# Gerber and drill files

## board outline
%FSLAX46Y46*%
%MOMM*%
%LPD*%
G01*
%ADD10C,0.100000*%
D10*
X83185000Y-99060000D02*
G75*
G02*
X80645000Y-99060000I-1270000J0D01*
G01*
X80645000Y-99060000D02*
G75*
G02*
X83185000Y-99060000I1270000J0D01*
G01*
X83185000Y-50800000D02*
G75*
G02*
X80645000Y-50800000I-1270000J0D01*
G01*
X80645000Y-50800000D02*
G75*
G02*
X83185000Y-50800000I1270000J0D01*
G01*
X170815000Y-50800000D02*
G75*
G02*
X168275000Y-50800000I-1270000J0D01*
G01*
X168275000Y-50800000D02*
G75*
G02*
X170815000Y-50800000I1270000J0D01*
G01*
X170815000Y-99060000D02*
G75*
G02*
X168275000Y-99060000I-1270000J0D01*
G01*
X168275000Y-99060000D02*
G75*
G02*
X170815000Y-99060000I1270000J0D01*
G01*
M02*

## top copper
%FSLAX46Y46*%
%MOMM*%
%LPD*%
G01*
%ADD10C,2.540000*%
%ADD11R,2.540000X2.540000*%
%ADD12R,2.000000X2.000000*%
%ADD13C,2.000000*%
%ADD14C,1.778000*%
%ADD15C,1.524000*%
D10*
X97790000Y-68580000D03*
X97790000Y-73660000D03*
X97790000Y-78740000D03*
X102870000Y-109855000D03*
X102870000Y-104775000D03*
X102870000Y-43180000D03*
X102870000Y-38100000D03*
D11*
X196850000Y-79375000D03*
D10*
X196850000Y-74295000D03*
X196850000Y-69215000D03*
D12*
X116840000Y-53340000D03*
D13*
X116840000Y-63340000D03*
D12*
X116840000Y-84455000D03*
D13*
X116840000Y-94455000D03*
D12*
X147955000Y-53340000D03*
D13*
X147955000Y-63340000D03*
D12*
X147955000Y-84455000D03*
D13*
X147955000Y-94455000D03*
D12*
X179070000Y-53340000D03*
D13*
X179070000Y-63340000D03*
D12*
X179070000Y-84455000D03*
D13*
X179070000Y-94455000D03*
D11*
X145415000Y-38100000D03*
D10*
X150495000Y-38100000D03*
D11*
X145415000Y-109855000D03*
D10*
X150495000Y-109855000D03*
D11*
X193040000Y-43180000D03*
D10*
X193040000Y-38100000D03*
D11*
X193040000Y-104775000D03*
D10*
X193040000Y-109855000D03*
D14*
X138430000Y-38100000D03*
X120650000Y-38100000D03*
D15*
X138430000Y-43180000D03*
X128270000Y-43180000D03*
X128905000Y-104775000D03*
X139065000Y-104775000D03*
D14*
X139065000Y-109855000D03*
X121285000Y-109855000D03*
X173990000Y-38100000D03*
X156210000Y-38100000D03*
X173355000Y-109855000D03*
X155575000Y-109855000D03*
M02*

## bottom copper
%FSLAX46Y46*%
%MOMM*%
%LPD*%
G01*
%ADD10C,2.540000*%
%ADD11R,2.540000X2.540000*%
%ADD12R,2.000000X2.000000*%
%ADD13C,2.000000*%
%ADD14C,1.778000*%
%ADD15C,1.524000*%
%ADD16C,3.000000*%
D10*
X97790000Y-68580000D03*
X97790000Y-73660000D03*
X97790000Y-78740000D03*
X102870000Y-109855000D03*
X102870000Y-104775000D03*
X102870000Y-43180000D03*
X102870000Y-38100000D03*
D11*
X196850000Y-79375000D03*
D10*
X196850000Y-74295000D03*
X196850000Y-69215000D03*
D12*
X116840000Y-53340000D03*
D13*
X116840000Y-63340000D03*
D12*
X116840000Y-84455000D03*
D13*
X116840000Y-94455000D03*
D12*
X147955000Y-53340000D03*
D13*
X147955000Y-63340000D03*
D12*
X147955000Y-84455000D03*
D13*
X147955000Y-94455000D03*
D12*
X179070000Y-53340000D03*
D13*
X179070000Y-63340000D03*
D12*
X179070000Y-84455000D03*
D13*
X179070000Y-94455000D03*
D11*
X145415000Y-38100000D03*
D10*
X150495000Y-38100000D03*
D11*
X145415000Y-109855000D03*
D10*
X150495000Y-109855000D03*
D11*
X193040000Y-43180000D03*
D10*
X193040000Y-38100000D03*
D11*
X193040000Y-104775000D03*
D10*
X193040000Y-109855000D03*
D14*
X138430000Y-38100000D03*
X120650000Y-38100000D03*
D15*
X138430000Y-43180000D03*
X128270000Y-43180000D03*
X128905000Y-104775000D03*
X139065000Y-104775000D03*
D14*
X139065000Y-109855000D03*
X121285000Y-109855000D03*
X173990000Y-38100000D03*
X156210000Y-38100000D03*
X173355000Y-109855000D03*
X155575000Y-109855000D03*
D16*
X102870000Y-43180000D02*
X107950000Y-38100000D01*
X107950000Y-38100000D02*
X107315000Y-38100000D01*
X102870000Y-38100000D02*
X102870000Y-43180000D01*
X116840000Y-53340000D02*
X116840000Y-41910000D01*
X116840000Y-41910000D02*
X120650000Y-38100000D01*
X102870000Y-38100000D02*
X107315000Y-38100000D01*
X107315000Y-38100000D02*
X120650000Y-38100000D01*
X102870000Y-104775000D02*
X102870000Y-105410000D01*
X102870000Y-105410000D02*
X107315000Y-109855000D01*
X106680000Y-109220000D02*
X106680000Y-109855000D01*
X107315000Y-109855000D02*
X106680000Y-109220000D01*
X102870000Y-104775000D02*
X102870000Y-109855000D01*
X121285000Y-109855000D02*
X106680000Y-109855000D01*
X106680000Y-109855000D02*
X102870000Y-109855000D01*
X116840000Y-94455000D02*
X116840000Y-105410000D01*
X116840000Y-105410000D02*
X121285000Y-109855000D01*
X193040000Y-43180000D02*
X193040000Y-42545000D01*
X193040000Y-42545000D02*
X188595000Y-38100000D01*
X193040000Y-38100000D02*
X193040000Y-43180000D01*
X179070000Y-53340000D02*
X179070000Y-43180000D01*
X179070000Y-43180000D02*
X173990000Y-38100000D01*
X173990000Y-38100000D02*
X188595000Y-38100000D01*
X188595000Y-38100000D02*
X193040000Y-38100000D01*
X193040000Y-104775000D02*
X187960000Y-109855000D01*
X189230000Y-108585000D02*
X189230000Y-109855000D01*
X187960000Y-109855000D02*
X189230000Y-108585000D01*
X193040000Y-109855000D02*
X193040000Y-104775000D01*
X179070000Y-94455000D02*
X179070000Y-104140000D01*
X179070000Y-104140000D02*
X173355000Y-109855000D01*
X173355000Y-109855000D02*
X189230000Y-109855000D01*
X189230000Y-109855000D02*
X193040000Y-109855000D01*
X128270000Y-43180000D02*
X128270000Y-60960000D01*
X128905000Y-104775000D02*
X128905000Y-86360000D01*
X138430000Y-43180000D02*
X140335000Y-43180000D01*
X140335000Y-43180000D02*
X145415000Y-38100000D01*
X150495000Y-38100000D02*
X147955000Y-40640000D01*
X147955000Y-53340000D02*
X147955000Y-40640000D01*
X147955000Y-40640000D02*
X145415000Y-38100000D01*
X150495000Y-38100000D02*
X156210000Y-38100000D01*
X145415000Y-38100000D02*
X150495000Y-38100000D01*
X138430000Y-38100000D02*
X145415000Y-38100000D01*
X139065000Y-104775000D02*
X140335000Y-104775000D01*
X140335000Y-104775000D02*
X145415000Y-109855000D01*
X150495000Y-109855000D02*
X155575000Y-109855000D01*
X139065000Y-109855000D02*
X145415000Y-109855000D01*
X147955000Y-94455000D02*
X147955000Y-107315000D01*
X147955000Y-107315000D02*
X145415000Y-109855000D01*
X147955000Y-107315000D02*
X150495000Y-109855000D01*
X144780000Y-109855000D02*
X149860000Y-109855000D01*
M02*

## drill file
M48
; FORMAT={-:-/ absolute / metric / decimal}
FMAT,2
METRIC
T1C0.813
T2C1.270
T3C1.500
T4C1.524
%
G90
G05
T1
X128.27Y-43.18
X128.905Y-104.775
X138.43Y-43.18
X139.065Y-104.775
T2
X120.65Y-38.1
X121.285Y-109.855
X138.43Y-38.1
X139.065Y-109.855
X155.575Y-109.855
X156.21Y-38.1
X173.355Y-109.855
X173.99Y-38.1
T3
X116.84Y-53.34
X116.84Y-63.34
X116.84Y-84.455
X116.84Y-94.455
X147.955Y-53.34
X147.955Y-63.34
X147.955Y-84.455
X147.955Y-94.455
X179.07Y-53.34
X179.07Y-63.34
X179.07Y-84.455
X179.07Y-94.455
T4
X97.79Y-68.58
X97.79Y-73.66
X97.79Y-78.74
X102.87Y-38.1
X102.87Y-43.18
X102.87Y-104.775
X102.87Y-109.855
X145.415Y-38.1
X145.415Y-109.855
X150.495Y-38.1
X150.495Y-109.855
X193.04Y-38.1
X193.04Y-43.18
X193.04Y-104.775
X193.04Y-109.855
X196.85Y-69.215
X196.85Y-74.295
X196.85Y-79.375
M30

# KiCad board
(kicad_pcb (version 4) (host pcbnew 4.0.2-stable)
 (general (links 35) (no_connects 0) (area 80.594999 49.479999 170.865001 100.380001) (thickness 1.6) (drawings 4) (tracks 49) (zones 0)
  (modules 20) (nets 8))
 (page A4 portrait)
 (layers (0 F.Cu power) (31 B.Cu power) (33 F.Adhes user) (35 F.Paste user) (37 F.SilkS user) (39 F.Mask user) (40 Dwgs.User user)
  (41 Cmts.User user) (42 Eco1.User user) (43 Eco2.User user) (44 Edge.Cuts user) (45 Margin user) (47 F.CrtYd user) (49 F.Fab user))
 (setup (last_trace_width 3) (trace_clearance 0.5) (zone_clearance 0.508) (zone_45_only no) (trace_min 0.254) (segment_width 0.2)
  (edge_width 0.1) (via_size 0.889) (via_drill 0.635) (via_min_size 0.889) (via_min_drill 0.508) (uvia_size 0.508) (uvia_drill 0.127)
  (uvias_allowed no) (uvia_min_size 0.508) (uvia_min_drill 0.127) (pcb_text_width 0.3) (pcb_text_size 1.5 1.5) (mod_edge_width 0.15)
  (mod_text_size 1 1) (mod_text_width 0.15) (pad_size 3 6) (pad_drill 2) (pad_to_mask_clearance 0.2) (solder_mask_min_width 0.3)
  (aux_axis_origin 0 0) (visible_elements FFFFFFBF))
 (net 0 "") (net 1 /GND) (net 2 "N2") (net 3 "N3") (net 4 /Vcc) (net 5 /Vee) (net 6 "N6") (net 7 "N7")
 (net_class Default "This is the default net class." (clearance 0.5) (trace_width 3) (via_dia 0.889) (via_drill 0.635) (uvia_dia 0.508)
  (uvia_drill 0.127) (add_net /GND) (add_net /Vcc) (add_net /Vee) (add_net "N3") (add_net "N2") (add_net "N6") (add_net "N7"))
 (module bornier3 (layer F.Cu) (at 97.79 73.66 270)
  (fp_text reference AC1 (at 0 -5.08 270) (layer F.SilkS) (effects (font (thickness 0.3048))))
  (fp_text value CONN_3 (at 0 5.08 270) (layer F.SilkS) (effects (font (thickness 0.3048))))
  (pad 1 thru_hole circle (at -5.08 0 270) (size 2.54 2.54) (drill 1.524) (layers *.Cu *.Mask F.SilkS) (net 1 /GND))
  (pad 2 thru_hole circle (at 0 0 270) (size 2.54 2.54) (drill 1.524) (layers *.Cu *.Mask F.SilkS) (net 1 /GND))
  (pad 3 thru_hole circle (at 5.08 0 270) (size 2.54 2.54) (drill 1.524) (layers *.Cu *.Mask F.SilkS) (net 1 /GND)))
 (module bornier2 (layer F.Cu) (at 102.87 107.315 90)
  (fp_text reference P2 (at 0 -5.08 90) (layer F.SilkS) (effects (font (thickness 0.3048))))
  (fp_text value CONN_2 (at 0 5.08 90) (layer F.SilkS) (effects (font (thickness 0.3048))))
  (pad 1 thru_hole circle (at -2.54 0 90) (size 2.54 2.54) (drill 1.524) (layers *.Cu *.Mask F.SilkS) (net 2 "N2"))
  (pad 2 thru_hole circle (at 2.54 0 90) (size 2.54 2.54) (drill 1.524) (layers *.Cu *.Mask F.SilkS) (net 2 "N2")))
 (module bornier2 (layer F.Cu) (at 102.87 40.64 90)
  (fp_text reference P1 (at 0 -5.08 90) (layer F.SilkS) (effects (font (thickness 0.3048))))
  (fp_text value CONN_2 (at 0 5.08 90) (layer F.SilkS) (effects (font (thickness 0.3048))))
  (pad 1 thru_hole circle (at -2.54 0 90) (size 2.54 2.54) (drill 1.524) (layers *.Cu *.Mask F.SilkS) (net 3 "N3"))
  (pad 2 thru_hole circle (at 2.54 0 90) (size 2.54 2.54) (drill 1.524) (layers *.Cu *.Mask F.SilkS) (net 3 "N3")))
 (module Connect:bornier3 (layer F.Cu) (at 196.85 74.295 90)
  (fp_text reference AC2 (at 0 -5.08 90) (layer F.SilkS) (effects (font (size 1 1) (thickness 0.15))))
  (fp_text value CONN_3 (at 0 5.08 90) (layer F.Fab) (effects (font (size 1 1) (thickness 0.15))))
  (pad 1 thru_hole rect (at -5.08 0 90) (size 2.54 2.54) (drill 1.524) (layers *.Cu *.Mask F.SilkS) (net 1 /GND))
  (pad 2 thru_hole circle (at 0 0 90) (size 2.54 2.54) (drill 1.524) (layers *.Cu *.Mask F.SilkS) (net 1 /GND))
  (pad 3 thru_hole circle (at 5.08 0 90) (size 2.54 2.54) (drill 1.524) (layers *.Cu *.Mask F.SilkS) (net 1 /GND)))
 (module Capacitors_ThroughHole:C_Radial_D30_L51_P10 (layer F.Cu) (at 116.84 53.34 270)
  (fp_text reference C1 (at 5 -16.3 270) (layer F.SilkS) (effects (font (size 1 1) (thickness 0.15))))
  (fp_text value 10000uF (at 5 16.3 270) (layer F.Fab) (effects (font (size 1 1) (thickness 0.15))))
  (pad 1 thru_hole rect (at 0 0 270) (size 2 2) (drill 1.5) (layers *.Cu *.Mask F.SilkS) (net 3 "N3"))
  (pad 2 thru_hole circle (at 10 0 270) (size 2 2) (drill 1.5) (layers *.Cu *.Mask F.SilkS) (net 1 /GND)))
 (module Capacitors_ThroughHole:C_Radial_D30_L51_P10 (layer F.Cu) (at 116.84 84.455 270)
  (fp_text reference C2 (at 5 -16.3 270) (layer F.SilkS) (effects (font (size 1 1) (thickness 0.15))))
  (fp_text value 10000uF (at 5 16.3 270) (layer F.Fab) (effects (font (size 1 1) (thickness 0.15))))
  (pad 1 thru_hole rect (at 0 0 270) (size 2 2) (drill 1.5) (layers *.Cu *.Mask F.SilkS) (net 1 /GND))
  (pad 2 thru_hole circle (at 10 0 270) (size 2 2) (drill 1.5) (layers *.Cu *.Mask F.SilkS) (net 2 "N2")))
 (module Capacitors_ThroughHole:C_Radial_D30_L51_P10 (layer F.Cu) (at 147.955 53.34 270)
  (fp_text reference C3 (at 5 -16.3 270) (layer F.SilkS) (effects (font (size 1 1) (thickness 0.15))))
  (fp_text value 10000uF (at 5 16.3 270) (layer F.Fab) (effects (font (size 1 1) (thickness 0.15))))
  (pad 1 thru_hole rect (at 0 0 270) (size 2 2) (drill 1.5) (layers *.Cu *.Mask F.SilkS) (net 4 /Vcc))
  (pad 2 thru_hole circle (at 10 0 270) (size 2 2) (drill 1.5) (layers *.Cu *.Mask F.SilkS) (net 1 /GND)))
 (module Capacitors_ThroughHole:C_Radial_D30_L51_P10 (layer F.Cu) (at 147.955 84.455 270)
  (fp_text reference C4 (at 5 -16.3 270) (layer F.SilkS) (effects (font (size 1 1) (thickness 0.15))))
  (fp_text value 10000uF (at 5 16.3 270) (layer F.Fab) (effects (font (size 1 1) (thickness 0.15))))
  (pad 1 thru_hole rect (at 0 0 270) (size 2 2) (drill 1.5) (layers *.Cu *.Mask F.SilkS) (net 1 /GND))
  (pad 2 thru_hole circle (at 10 0 270) (size 2 2) (drill 1.5) (layers *.Cu *.Mask F.SilkS) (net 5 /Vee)))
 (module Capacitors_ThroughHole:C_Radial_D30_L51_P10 (layer F.Cu) (at 179.07 53.34 270)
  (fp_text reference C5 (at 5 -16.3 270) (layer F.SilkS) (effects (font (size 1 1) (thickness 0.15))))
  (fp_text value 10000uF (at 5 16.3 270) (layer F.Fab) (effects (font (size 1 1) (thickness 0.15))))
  (pad 1 thru_hole rect (at 0 0 270) (size 2 2) (drill 1.5) (layers *.Cu *.Mask F.SilkS) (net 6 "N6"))
  (pad 2 thru_hole circle (at 10 0 270) (size 2 2) (drill 1.5) (layers *.Cu *.Mask F.SilkS) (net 1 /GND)))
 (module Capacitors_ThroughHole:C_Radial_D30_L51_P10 (layer F.Cu) (at 179.07 84.455 270)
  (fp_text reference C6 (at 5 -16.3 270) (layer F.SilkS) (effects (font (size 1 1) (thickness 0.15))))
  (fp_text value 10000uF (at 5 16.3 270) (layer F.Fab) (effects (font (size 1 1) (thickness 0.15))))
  (pad 1 thru_hole rect (at 0 0 270) (size 2 2) (drill 1.5) (layers *.Cu *.Mask F.SilkS) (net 1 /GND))
  (pad 2 thru_hole circle (at 10 0 270) (size 2 2) (drill 1.5) (layers *.Cu *.Mask F.SilkS) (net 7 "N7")))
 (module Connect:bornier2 (layer F.Cu) (at 147.955 38.1)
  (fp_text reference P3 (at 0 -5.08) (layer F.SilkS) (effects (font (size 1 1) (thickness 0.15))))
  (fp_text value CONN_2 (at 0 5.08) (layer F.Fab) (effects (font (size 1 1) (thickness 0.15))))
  (pad 1 thru_hole rect (at -2.54 0) (size 2.54 2.54) (drill 1.524) (layers *.Cu *.Mask F.SilkS) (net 4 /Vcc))
  (pad 2 thru_hole circle (at 2.54 0) (size 2.54 2.54) (drill 1.524) (layers *.Cu *.Mask F.SilkS) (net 4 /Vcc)))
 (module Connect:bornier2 (layer F.Cu) (at 147.955 109.855)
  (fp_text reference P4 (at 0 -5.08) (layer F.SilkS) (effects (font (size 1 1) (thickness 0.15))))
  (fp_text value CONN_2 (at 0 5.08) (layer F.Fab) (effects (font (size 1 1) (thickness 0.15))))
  (pad 1 thru_hole rect (at -2.54 0) (size 2.54 2.54) (drill 1.524) (layers *.Cu *.Mask F.SilkS) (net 5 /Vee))
  (pad 2 thru_hole circle (at 2.54 0) (size 2.54 2.54) (drill 1.524) (layers *.Cu *.Mask F.SilkS) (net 5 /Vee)))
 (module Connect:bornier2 (layer F.Cu) (at 193.04 40.64 90)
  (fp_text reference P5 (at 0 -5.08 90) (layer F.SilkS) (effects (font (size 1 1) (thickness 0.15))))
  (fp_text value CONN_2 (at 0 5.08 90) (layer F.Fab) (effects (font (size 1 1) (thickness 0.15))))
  (pad 1 thru_hole rect (at -2.54 0 90) (size 2.54 2.54) (drill 1.524) (layers *.Cu *.Mask F.SilkS) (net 6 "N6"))
  (pad 2 thru_hole circle (at 2.54 0 90) (size 2.54 2.54) (drill 1.524) (layers *.Cu *.Mask F.SilkS) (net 6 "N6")))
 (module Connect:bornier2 (layer F.Cu) (at 193.04 107.315 270)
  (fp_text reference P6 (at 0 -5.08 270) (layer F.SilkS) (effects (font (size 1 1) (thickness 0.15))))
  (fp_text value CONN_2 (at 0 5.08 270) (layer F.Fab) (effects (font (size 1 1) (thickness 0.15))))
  (pad 1 thru_hole rect (at -2.54 0 270) (size 2.54 2.54) (drill 1.524) (layers *.Cu *.Mask F.SilkS) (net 7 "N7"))
  (pad 2 thru_hole circle (at 2.54 0 270) (size 2.54 2.54) (drill 1.524) (layers *.Cu *.Mask F.SilkS) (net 7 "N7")))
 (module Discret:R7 (layer F.Cu) (at 129.54 38.1 180)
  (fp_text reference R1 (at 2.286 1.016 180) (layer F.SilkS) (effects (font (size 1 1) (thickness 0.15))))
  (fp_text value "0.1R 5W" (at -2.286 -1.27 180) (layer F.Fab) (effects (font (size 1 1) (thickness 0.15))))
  (pad 1 thru_hole circle (at -8.89 0 180) (size 1.778 1.778) (drill 1.27) (layers *.Cu *.Mask F.SilkS) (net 4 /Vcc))
  (pad 2 thru_hole circle (at 8.89 0 180) (size 1.778 1.778) (drill 1.27) (layers *.Cu *.Mask F.SilkS) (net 3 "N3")))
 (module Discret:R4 (layer F.Cu) (at 133.35 43.18 180)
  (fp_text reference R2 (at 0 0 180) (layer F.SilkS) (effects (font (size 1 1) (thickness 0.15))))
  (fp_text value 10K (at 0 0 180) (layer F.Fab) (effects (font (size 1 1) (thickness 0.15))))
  (pad 1 thru_hole circle (at -5.08 0 180) (size 1.524 1.524) (drill 0.8128) (layers *.Cu *.Mask F.SilkS) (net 4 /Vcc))
  (pad 2 thru_hole circle (at 5.08 0 180) (size 1.524 1.524) (drill 0.8128) (layers *.Cu *.Mask F.SilkS) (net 1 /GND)))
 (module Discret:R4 (layer F.Cu) (at 133.985 104.775)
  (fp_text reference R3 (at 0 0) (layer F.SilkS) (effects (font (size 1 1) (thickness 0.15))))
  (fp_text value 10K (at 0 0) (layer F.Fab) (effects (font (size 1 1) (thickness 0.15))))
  (pad 1 thru_hole circle (at -5.08 0) (size 1.524 1.524) (drill 0.8128) (layers *.Cu *.Mask F.SilkS) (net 1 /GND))
  (pad 2 thru_hole circle (at 5.08 0) (size 1.524 1.524) (drill 0.8128) (layers *.Cu *.Mask F.SilkS) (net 5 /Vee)))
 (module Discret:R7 (layer F.Cu) (at 130.175 109.855 180)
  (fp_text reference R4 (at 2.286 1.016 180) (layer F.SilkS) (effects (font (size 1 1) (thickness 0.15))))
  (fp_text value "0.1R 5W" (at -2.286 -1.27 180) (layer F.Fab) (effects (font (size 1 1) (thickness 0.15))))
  (pad 1 thru_hole circle (at -8.89 0 180) (size 1.778 1.778) (drill 1.27) (layers *.Cu *.Mask F.SilkS) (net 5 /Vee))
  (pad 2 thru_hole circle (at 8.89 0 180) (size 1.778 1.778) (drill 1.27) (layers *.Cu *.Mask F.SilkS) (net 2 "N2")))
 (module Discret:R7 (layer F.Cu) (at 165.1 38.1 180)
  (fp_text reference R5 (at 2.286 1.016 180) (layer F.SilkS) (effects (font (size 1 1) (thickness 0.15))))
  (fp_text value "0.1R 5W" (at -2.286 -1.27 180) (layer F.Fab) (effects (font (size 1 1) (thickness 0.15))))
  (pad 1 thru_hole circle (at -8.89 0 180) (size 1.778 1.778) (drill 1.27) (layers *.Cu *.Mask F.SilkS) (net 6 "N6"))
  (pad 2 thru_hole circle (at 8.89 0 180) (size 1.778 1.778) (drill 1.27) (layers *.Cu *.Mask F.SilkS) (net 4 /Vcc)))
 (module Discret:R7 (layer F.Cu) (at 164.465 109.855 180)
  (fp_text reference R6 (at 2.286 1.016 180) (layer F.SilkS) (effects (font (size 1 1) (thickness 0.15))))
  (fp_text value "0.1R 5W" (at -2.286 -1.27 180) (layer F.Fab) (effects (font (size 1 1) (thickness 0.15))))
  (pad 1 thru_hole circle (at -8.89 0 180) (size 1.778 1.778) (drill 1.27) (layers *.Cu *.Mask F.SilkS) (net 7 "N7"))
  (pad 2 thru_hole circle (at 8.89 0 180) (size 1.778 1.778) (drill 1.27) (layers *.Cu *.Mask F.SilkS) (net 5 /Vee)))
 (gr_circle (center 81.915 99.06) (end 83.185 99.06) (layer Edge.Cuts) (width 0.1))
 (gr_circle (center 81.915 50.8) (end 83.185 50.8) (layer Edge.Cuts) (width 0.1))
 (gr_circle (center 169.545 50.8) (end 170.815 50.8) (layer Edge.Cuts) (width 0.1))
 (gr_circle (center 169.545 99.06) (end 170.815 99.06) (layer Edge.Cuts) (width 0.1))
 (segment (start 102.87 43.18) (end 107.95 38.1) (width 3) (layer B.Cu) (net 3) (status 400000))
 (segment (start 107.95 38.1) (end 107.315 38.1) (width 3) (layer B.Cu) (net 3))
 (segment (start 102.87 38.1) (end 102.87 43.18) (width 3) (layer B.Cu) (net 3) (status C00000))
 (segment (start 116.84 53.34) (end 116.84 41.91) (width 3) (layer B.Cu) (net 3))
 (segment (start 116.84 41.91) (end 120.65 38.1) (width 3) (layer B.Cu) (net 3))
 (segment (start 102.87 38.1) (end 107.315 38.1) (width 3) (layer B.Cu) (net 3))
 (segment (start 107.315 38.1) (end 120.65 38.1) (width 3) (layer B.Cu) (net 3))
 (segment (start 102.87 104.775) (end 102.87 105.41) (width 3) (layer B.Cu) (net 2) (status C00000))
 (segment (start 102.87 105.41) (end 107.315 109.855) (width 3) (layer B.Cu) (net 2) (status 400000))
 (segment (start 106.68 109.22) (end 106.68 109.855) (width 3) (layer B.Cu) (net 2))
 (segment (start 107.315 109.855) (end 106.68 109.22) (width 3) (layer B.Cu) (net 2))
 (segment (start 102.87 104.775) (end 102.87 109.855) (width 3) (layer B.Cu) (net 2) (status C00000))
 (segment (start 121.285 109.855) (end 106.68 109.855) (width 3) (layer B.Cu) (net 2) (status 400000))
 (segment (start 106.68 109.855) (end 102.87 109.855) (width 3) (layer B.Cu) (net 2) (status 800000))
 (segment (start 116.84 94.455) (end 116.84 105.41) (width 3) (layer B.Cu) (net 2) (status 400000))
 (segment (start 116.84 105.41) (end 121.285 109.855) (width 3) (layer B.Cu) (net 2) (status 800000))
 (segment (start 193.04 43.18) (end 193.04 42.545) (width 3) (layer B.Cu) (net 6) (status C00000))
 (segment (start 193.04 42.545) (end 188.595 38.1) (width 3) (layer B.Cu) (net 6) (status 400000))
 (segment (start 193.04 38.1) (end 193.04 43.18) (width 3) (layer B.Cu) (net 6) (status C00000))
 (segment (start 179.07 53.34) (end 179.07 43.18) (width 3) (layer B.Cu) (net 6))
 (segment (start 179.07 43.18) (end 173.99 38.1) (width 3) (layer B.Cu) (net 6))
 (segment (start 173.99 38.1) (end 188.595 38.1) (width 3) (layer B.Cu) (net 6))
 (segment (start 188.595 38.1) (end 193.04 38.1) (width 3) (layer B.Cu) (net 6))
 (segment (start 193.04 104.775) (end 187.96 109.855) (width 3) (layer B.Cu) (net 7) (status 400000))
 (segment (start 189.23 108.585) (end 189.23 109.855) (width 3) (layer B.Cu) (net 7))
 (segment (start 187.96 109.855) (end 189.23 108.585) (width 3) (layer B.Cu) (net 7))
 (segment (start 193.04 109.855) (end 193.04 104.775) (width 3) (layer B.Cu) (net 7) (status C00000))
 (segment (start 179.07 94.455) (end 179.07 104.14) (width 3) (layer B.Cu) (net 7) (status 400000))
 (segment (start 179.07 104.14) (end 173.355 109.855) (width 3) (layer B.Cu) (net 7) (status 800000))
 (segment (start 173.355 109.855) (end 189.23 109.855) (width 3) (layer B.Cu) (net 7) (status 400000))
 (segment (start 189.23 109.855) (end 193.04 109.855) (width 3) (layer B.Cu) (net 7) (status 800000))
 (segment (start 128.27 43.18) (end 128.27 60.96) (width 3) (layer B.Cu) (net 1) (status 400000))
 (segment (start 128.905 104.775) (end 128.905 86.36) (width 3) (layer B.Cu) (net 1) (status 400000))
 (segment (start 138.43 43.18) (end 140.335 43.18) (width 3) (layer B.Cu) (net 4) (status 400000))
 (segment (start 140.335 43.18) (end 145.415 38.1) (width 3) (layer B.Cu) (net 4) (status 800000))
 (segment (start 150.495 38.1) (end 147.955 40.64) (width 3) (layer B.Cu) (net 4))
 (segment (start 147.955 53.34) (end 147.955 40.64) (width 3) (layer B.Cu) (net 4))
 (segment (start 147.955 40.64) (end 145.415 38.1) (width 3) (layer B.Cu) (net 4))
 (segment (start 150.495 38.1) (end 156.21 38.1) (width 3) (layer B.Cu) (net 4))
 (segment (start 145.415 38.1) (end 150.495 38.1) (width 3) (layer B.Cu) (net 4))
 (segment (start 138.43 38.1) (end 145.415 38.1) (width 3) (layer B.Cu) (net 4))
 (segment (start 139.065 104.775) (end 140.335 104.775) (width 3) (layer B.Cu) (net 5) (status 400000))
 (segment (start 140.335 104.775) (end 145.415 109.855) (width 3) (layer B.Cu) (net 5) (status 800000))
 (segment (start 150.495 109.855) (end 155.575 109.855) (width 3) (layer B.Cu) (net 5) (status C00000))
 (segment (start 139.065 109.855) (end 145.415 109.855) (width 3) (layer B.Cu) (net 5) (status C00000))
 (segment (start 147.955 94.455) (end 147.955 107.315) (width 3) (layer B.Cu) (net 5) (status 400000))
 (segment (start 147.955 107.315) (end 145.415 109.855) (width 3) (layer B.Cu) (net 5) (status 800000))
 (segment (start 147.955 107.315) (end 150.495 109.855) (width 3) (layer B.Cu) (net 5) (status 800000))
 (segment (start 144.78 109.855) (end 149.86 109.855) (width 3) (layer B.Cu) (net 5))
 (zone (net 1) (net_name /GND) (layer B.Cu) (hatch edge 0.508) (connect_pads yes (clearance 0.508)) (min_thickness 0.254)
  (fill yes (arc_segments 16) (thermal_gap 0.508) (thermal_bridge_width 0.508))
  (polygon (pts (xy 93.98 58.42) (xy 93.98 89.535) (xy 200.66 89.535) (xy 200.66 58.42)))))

